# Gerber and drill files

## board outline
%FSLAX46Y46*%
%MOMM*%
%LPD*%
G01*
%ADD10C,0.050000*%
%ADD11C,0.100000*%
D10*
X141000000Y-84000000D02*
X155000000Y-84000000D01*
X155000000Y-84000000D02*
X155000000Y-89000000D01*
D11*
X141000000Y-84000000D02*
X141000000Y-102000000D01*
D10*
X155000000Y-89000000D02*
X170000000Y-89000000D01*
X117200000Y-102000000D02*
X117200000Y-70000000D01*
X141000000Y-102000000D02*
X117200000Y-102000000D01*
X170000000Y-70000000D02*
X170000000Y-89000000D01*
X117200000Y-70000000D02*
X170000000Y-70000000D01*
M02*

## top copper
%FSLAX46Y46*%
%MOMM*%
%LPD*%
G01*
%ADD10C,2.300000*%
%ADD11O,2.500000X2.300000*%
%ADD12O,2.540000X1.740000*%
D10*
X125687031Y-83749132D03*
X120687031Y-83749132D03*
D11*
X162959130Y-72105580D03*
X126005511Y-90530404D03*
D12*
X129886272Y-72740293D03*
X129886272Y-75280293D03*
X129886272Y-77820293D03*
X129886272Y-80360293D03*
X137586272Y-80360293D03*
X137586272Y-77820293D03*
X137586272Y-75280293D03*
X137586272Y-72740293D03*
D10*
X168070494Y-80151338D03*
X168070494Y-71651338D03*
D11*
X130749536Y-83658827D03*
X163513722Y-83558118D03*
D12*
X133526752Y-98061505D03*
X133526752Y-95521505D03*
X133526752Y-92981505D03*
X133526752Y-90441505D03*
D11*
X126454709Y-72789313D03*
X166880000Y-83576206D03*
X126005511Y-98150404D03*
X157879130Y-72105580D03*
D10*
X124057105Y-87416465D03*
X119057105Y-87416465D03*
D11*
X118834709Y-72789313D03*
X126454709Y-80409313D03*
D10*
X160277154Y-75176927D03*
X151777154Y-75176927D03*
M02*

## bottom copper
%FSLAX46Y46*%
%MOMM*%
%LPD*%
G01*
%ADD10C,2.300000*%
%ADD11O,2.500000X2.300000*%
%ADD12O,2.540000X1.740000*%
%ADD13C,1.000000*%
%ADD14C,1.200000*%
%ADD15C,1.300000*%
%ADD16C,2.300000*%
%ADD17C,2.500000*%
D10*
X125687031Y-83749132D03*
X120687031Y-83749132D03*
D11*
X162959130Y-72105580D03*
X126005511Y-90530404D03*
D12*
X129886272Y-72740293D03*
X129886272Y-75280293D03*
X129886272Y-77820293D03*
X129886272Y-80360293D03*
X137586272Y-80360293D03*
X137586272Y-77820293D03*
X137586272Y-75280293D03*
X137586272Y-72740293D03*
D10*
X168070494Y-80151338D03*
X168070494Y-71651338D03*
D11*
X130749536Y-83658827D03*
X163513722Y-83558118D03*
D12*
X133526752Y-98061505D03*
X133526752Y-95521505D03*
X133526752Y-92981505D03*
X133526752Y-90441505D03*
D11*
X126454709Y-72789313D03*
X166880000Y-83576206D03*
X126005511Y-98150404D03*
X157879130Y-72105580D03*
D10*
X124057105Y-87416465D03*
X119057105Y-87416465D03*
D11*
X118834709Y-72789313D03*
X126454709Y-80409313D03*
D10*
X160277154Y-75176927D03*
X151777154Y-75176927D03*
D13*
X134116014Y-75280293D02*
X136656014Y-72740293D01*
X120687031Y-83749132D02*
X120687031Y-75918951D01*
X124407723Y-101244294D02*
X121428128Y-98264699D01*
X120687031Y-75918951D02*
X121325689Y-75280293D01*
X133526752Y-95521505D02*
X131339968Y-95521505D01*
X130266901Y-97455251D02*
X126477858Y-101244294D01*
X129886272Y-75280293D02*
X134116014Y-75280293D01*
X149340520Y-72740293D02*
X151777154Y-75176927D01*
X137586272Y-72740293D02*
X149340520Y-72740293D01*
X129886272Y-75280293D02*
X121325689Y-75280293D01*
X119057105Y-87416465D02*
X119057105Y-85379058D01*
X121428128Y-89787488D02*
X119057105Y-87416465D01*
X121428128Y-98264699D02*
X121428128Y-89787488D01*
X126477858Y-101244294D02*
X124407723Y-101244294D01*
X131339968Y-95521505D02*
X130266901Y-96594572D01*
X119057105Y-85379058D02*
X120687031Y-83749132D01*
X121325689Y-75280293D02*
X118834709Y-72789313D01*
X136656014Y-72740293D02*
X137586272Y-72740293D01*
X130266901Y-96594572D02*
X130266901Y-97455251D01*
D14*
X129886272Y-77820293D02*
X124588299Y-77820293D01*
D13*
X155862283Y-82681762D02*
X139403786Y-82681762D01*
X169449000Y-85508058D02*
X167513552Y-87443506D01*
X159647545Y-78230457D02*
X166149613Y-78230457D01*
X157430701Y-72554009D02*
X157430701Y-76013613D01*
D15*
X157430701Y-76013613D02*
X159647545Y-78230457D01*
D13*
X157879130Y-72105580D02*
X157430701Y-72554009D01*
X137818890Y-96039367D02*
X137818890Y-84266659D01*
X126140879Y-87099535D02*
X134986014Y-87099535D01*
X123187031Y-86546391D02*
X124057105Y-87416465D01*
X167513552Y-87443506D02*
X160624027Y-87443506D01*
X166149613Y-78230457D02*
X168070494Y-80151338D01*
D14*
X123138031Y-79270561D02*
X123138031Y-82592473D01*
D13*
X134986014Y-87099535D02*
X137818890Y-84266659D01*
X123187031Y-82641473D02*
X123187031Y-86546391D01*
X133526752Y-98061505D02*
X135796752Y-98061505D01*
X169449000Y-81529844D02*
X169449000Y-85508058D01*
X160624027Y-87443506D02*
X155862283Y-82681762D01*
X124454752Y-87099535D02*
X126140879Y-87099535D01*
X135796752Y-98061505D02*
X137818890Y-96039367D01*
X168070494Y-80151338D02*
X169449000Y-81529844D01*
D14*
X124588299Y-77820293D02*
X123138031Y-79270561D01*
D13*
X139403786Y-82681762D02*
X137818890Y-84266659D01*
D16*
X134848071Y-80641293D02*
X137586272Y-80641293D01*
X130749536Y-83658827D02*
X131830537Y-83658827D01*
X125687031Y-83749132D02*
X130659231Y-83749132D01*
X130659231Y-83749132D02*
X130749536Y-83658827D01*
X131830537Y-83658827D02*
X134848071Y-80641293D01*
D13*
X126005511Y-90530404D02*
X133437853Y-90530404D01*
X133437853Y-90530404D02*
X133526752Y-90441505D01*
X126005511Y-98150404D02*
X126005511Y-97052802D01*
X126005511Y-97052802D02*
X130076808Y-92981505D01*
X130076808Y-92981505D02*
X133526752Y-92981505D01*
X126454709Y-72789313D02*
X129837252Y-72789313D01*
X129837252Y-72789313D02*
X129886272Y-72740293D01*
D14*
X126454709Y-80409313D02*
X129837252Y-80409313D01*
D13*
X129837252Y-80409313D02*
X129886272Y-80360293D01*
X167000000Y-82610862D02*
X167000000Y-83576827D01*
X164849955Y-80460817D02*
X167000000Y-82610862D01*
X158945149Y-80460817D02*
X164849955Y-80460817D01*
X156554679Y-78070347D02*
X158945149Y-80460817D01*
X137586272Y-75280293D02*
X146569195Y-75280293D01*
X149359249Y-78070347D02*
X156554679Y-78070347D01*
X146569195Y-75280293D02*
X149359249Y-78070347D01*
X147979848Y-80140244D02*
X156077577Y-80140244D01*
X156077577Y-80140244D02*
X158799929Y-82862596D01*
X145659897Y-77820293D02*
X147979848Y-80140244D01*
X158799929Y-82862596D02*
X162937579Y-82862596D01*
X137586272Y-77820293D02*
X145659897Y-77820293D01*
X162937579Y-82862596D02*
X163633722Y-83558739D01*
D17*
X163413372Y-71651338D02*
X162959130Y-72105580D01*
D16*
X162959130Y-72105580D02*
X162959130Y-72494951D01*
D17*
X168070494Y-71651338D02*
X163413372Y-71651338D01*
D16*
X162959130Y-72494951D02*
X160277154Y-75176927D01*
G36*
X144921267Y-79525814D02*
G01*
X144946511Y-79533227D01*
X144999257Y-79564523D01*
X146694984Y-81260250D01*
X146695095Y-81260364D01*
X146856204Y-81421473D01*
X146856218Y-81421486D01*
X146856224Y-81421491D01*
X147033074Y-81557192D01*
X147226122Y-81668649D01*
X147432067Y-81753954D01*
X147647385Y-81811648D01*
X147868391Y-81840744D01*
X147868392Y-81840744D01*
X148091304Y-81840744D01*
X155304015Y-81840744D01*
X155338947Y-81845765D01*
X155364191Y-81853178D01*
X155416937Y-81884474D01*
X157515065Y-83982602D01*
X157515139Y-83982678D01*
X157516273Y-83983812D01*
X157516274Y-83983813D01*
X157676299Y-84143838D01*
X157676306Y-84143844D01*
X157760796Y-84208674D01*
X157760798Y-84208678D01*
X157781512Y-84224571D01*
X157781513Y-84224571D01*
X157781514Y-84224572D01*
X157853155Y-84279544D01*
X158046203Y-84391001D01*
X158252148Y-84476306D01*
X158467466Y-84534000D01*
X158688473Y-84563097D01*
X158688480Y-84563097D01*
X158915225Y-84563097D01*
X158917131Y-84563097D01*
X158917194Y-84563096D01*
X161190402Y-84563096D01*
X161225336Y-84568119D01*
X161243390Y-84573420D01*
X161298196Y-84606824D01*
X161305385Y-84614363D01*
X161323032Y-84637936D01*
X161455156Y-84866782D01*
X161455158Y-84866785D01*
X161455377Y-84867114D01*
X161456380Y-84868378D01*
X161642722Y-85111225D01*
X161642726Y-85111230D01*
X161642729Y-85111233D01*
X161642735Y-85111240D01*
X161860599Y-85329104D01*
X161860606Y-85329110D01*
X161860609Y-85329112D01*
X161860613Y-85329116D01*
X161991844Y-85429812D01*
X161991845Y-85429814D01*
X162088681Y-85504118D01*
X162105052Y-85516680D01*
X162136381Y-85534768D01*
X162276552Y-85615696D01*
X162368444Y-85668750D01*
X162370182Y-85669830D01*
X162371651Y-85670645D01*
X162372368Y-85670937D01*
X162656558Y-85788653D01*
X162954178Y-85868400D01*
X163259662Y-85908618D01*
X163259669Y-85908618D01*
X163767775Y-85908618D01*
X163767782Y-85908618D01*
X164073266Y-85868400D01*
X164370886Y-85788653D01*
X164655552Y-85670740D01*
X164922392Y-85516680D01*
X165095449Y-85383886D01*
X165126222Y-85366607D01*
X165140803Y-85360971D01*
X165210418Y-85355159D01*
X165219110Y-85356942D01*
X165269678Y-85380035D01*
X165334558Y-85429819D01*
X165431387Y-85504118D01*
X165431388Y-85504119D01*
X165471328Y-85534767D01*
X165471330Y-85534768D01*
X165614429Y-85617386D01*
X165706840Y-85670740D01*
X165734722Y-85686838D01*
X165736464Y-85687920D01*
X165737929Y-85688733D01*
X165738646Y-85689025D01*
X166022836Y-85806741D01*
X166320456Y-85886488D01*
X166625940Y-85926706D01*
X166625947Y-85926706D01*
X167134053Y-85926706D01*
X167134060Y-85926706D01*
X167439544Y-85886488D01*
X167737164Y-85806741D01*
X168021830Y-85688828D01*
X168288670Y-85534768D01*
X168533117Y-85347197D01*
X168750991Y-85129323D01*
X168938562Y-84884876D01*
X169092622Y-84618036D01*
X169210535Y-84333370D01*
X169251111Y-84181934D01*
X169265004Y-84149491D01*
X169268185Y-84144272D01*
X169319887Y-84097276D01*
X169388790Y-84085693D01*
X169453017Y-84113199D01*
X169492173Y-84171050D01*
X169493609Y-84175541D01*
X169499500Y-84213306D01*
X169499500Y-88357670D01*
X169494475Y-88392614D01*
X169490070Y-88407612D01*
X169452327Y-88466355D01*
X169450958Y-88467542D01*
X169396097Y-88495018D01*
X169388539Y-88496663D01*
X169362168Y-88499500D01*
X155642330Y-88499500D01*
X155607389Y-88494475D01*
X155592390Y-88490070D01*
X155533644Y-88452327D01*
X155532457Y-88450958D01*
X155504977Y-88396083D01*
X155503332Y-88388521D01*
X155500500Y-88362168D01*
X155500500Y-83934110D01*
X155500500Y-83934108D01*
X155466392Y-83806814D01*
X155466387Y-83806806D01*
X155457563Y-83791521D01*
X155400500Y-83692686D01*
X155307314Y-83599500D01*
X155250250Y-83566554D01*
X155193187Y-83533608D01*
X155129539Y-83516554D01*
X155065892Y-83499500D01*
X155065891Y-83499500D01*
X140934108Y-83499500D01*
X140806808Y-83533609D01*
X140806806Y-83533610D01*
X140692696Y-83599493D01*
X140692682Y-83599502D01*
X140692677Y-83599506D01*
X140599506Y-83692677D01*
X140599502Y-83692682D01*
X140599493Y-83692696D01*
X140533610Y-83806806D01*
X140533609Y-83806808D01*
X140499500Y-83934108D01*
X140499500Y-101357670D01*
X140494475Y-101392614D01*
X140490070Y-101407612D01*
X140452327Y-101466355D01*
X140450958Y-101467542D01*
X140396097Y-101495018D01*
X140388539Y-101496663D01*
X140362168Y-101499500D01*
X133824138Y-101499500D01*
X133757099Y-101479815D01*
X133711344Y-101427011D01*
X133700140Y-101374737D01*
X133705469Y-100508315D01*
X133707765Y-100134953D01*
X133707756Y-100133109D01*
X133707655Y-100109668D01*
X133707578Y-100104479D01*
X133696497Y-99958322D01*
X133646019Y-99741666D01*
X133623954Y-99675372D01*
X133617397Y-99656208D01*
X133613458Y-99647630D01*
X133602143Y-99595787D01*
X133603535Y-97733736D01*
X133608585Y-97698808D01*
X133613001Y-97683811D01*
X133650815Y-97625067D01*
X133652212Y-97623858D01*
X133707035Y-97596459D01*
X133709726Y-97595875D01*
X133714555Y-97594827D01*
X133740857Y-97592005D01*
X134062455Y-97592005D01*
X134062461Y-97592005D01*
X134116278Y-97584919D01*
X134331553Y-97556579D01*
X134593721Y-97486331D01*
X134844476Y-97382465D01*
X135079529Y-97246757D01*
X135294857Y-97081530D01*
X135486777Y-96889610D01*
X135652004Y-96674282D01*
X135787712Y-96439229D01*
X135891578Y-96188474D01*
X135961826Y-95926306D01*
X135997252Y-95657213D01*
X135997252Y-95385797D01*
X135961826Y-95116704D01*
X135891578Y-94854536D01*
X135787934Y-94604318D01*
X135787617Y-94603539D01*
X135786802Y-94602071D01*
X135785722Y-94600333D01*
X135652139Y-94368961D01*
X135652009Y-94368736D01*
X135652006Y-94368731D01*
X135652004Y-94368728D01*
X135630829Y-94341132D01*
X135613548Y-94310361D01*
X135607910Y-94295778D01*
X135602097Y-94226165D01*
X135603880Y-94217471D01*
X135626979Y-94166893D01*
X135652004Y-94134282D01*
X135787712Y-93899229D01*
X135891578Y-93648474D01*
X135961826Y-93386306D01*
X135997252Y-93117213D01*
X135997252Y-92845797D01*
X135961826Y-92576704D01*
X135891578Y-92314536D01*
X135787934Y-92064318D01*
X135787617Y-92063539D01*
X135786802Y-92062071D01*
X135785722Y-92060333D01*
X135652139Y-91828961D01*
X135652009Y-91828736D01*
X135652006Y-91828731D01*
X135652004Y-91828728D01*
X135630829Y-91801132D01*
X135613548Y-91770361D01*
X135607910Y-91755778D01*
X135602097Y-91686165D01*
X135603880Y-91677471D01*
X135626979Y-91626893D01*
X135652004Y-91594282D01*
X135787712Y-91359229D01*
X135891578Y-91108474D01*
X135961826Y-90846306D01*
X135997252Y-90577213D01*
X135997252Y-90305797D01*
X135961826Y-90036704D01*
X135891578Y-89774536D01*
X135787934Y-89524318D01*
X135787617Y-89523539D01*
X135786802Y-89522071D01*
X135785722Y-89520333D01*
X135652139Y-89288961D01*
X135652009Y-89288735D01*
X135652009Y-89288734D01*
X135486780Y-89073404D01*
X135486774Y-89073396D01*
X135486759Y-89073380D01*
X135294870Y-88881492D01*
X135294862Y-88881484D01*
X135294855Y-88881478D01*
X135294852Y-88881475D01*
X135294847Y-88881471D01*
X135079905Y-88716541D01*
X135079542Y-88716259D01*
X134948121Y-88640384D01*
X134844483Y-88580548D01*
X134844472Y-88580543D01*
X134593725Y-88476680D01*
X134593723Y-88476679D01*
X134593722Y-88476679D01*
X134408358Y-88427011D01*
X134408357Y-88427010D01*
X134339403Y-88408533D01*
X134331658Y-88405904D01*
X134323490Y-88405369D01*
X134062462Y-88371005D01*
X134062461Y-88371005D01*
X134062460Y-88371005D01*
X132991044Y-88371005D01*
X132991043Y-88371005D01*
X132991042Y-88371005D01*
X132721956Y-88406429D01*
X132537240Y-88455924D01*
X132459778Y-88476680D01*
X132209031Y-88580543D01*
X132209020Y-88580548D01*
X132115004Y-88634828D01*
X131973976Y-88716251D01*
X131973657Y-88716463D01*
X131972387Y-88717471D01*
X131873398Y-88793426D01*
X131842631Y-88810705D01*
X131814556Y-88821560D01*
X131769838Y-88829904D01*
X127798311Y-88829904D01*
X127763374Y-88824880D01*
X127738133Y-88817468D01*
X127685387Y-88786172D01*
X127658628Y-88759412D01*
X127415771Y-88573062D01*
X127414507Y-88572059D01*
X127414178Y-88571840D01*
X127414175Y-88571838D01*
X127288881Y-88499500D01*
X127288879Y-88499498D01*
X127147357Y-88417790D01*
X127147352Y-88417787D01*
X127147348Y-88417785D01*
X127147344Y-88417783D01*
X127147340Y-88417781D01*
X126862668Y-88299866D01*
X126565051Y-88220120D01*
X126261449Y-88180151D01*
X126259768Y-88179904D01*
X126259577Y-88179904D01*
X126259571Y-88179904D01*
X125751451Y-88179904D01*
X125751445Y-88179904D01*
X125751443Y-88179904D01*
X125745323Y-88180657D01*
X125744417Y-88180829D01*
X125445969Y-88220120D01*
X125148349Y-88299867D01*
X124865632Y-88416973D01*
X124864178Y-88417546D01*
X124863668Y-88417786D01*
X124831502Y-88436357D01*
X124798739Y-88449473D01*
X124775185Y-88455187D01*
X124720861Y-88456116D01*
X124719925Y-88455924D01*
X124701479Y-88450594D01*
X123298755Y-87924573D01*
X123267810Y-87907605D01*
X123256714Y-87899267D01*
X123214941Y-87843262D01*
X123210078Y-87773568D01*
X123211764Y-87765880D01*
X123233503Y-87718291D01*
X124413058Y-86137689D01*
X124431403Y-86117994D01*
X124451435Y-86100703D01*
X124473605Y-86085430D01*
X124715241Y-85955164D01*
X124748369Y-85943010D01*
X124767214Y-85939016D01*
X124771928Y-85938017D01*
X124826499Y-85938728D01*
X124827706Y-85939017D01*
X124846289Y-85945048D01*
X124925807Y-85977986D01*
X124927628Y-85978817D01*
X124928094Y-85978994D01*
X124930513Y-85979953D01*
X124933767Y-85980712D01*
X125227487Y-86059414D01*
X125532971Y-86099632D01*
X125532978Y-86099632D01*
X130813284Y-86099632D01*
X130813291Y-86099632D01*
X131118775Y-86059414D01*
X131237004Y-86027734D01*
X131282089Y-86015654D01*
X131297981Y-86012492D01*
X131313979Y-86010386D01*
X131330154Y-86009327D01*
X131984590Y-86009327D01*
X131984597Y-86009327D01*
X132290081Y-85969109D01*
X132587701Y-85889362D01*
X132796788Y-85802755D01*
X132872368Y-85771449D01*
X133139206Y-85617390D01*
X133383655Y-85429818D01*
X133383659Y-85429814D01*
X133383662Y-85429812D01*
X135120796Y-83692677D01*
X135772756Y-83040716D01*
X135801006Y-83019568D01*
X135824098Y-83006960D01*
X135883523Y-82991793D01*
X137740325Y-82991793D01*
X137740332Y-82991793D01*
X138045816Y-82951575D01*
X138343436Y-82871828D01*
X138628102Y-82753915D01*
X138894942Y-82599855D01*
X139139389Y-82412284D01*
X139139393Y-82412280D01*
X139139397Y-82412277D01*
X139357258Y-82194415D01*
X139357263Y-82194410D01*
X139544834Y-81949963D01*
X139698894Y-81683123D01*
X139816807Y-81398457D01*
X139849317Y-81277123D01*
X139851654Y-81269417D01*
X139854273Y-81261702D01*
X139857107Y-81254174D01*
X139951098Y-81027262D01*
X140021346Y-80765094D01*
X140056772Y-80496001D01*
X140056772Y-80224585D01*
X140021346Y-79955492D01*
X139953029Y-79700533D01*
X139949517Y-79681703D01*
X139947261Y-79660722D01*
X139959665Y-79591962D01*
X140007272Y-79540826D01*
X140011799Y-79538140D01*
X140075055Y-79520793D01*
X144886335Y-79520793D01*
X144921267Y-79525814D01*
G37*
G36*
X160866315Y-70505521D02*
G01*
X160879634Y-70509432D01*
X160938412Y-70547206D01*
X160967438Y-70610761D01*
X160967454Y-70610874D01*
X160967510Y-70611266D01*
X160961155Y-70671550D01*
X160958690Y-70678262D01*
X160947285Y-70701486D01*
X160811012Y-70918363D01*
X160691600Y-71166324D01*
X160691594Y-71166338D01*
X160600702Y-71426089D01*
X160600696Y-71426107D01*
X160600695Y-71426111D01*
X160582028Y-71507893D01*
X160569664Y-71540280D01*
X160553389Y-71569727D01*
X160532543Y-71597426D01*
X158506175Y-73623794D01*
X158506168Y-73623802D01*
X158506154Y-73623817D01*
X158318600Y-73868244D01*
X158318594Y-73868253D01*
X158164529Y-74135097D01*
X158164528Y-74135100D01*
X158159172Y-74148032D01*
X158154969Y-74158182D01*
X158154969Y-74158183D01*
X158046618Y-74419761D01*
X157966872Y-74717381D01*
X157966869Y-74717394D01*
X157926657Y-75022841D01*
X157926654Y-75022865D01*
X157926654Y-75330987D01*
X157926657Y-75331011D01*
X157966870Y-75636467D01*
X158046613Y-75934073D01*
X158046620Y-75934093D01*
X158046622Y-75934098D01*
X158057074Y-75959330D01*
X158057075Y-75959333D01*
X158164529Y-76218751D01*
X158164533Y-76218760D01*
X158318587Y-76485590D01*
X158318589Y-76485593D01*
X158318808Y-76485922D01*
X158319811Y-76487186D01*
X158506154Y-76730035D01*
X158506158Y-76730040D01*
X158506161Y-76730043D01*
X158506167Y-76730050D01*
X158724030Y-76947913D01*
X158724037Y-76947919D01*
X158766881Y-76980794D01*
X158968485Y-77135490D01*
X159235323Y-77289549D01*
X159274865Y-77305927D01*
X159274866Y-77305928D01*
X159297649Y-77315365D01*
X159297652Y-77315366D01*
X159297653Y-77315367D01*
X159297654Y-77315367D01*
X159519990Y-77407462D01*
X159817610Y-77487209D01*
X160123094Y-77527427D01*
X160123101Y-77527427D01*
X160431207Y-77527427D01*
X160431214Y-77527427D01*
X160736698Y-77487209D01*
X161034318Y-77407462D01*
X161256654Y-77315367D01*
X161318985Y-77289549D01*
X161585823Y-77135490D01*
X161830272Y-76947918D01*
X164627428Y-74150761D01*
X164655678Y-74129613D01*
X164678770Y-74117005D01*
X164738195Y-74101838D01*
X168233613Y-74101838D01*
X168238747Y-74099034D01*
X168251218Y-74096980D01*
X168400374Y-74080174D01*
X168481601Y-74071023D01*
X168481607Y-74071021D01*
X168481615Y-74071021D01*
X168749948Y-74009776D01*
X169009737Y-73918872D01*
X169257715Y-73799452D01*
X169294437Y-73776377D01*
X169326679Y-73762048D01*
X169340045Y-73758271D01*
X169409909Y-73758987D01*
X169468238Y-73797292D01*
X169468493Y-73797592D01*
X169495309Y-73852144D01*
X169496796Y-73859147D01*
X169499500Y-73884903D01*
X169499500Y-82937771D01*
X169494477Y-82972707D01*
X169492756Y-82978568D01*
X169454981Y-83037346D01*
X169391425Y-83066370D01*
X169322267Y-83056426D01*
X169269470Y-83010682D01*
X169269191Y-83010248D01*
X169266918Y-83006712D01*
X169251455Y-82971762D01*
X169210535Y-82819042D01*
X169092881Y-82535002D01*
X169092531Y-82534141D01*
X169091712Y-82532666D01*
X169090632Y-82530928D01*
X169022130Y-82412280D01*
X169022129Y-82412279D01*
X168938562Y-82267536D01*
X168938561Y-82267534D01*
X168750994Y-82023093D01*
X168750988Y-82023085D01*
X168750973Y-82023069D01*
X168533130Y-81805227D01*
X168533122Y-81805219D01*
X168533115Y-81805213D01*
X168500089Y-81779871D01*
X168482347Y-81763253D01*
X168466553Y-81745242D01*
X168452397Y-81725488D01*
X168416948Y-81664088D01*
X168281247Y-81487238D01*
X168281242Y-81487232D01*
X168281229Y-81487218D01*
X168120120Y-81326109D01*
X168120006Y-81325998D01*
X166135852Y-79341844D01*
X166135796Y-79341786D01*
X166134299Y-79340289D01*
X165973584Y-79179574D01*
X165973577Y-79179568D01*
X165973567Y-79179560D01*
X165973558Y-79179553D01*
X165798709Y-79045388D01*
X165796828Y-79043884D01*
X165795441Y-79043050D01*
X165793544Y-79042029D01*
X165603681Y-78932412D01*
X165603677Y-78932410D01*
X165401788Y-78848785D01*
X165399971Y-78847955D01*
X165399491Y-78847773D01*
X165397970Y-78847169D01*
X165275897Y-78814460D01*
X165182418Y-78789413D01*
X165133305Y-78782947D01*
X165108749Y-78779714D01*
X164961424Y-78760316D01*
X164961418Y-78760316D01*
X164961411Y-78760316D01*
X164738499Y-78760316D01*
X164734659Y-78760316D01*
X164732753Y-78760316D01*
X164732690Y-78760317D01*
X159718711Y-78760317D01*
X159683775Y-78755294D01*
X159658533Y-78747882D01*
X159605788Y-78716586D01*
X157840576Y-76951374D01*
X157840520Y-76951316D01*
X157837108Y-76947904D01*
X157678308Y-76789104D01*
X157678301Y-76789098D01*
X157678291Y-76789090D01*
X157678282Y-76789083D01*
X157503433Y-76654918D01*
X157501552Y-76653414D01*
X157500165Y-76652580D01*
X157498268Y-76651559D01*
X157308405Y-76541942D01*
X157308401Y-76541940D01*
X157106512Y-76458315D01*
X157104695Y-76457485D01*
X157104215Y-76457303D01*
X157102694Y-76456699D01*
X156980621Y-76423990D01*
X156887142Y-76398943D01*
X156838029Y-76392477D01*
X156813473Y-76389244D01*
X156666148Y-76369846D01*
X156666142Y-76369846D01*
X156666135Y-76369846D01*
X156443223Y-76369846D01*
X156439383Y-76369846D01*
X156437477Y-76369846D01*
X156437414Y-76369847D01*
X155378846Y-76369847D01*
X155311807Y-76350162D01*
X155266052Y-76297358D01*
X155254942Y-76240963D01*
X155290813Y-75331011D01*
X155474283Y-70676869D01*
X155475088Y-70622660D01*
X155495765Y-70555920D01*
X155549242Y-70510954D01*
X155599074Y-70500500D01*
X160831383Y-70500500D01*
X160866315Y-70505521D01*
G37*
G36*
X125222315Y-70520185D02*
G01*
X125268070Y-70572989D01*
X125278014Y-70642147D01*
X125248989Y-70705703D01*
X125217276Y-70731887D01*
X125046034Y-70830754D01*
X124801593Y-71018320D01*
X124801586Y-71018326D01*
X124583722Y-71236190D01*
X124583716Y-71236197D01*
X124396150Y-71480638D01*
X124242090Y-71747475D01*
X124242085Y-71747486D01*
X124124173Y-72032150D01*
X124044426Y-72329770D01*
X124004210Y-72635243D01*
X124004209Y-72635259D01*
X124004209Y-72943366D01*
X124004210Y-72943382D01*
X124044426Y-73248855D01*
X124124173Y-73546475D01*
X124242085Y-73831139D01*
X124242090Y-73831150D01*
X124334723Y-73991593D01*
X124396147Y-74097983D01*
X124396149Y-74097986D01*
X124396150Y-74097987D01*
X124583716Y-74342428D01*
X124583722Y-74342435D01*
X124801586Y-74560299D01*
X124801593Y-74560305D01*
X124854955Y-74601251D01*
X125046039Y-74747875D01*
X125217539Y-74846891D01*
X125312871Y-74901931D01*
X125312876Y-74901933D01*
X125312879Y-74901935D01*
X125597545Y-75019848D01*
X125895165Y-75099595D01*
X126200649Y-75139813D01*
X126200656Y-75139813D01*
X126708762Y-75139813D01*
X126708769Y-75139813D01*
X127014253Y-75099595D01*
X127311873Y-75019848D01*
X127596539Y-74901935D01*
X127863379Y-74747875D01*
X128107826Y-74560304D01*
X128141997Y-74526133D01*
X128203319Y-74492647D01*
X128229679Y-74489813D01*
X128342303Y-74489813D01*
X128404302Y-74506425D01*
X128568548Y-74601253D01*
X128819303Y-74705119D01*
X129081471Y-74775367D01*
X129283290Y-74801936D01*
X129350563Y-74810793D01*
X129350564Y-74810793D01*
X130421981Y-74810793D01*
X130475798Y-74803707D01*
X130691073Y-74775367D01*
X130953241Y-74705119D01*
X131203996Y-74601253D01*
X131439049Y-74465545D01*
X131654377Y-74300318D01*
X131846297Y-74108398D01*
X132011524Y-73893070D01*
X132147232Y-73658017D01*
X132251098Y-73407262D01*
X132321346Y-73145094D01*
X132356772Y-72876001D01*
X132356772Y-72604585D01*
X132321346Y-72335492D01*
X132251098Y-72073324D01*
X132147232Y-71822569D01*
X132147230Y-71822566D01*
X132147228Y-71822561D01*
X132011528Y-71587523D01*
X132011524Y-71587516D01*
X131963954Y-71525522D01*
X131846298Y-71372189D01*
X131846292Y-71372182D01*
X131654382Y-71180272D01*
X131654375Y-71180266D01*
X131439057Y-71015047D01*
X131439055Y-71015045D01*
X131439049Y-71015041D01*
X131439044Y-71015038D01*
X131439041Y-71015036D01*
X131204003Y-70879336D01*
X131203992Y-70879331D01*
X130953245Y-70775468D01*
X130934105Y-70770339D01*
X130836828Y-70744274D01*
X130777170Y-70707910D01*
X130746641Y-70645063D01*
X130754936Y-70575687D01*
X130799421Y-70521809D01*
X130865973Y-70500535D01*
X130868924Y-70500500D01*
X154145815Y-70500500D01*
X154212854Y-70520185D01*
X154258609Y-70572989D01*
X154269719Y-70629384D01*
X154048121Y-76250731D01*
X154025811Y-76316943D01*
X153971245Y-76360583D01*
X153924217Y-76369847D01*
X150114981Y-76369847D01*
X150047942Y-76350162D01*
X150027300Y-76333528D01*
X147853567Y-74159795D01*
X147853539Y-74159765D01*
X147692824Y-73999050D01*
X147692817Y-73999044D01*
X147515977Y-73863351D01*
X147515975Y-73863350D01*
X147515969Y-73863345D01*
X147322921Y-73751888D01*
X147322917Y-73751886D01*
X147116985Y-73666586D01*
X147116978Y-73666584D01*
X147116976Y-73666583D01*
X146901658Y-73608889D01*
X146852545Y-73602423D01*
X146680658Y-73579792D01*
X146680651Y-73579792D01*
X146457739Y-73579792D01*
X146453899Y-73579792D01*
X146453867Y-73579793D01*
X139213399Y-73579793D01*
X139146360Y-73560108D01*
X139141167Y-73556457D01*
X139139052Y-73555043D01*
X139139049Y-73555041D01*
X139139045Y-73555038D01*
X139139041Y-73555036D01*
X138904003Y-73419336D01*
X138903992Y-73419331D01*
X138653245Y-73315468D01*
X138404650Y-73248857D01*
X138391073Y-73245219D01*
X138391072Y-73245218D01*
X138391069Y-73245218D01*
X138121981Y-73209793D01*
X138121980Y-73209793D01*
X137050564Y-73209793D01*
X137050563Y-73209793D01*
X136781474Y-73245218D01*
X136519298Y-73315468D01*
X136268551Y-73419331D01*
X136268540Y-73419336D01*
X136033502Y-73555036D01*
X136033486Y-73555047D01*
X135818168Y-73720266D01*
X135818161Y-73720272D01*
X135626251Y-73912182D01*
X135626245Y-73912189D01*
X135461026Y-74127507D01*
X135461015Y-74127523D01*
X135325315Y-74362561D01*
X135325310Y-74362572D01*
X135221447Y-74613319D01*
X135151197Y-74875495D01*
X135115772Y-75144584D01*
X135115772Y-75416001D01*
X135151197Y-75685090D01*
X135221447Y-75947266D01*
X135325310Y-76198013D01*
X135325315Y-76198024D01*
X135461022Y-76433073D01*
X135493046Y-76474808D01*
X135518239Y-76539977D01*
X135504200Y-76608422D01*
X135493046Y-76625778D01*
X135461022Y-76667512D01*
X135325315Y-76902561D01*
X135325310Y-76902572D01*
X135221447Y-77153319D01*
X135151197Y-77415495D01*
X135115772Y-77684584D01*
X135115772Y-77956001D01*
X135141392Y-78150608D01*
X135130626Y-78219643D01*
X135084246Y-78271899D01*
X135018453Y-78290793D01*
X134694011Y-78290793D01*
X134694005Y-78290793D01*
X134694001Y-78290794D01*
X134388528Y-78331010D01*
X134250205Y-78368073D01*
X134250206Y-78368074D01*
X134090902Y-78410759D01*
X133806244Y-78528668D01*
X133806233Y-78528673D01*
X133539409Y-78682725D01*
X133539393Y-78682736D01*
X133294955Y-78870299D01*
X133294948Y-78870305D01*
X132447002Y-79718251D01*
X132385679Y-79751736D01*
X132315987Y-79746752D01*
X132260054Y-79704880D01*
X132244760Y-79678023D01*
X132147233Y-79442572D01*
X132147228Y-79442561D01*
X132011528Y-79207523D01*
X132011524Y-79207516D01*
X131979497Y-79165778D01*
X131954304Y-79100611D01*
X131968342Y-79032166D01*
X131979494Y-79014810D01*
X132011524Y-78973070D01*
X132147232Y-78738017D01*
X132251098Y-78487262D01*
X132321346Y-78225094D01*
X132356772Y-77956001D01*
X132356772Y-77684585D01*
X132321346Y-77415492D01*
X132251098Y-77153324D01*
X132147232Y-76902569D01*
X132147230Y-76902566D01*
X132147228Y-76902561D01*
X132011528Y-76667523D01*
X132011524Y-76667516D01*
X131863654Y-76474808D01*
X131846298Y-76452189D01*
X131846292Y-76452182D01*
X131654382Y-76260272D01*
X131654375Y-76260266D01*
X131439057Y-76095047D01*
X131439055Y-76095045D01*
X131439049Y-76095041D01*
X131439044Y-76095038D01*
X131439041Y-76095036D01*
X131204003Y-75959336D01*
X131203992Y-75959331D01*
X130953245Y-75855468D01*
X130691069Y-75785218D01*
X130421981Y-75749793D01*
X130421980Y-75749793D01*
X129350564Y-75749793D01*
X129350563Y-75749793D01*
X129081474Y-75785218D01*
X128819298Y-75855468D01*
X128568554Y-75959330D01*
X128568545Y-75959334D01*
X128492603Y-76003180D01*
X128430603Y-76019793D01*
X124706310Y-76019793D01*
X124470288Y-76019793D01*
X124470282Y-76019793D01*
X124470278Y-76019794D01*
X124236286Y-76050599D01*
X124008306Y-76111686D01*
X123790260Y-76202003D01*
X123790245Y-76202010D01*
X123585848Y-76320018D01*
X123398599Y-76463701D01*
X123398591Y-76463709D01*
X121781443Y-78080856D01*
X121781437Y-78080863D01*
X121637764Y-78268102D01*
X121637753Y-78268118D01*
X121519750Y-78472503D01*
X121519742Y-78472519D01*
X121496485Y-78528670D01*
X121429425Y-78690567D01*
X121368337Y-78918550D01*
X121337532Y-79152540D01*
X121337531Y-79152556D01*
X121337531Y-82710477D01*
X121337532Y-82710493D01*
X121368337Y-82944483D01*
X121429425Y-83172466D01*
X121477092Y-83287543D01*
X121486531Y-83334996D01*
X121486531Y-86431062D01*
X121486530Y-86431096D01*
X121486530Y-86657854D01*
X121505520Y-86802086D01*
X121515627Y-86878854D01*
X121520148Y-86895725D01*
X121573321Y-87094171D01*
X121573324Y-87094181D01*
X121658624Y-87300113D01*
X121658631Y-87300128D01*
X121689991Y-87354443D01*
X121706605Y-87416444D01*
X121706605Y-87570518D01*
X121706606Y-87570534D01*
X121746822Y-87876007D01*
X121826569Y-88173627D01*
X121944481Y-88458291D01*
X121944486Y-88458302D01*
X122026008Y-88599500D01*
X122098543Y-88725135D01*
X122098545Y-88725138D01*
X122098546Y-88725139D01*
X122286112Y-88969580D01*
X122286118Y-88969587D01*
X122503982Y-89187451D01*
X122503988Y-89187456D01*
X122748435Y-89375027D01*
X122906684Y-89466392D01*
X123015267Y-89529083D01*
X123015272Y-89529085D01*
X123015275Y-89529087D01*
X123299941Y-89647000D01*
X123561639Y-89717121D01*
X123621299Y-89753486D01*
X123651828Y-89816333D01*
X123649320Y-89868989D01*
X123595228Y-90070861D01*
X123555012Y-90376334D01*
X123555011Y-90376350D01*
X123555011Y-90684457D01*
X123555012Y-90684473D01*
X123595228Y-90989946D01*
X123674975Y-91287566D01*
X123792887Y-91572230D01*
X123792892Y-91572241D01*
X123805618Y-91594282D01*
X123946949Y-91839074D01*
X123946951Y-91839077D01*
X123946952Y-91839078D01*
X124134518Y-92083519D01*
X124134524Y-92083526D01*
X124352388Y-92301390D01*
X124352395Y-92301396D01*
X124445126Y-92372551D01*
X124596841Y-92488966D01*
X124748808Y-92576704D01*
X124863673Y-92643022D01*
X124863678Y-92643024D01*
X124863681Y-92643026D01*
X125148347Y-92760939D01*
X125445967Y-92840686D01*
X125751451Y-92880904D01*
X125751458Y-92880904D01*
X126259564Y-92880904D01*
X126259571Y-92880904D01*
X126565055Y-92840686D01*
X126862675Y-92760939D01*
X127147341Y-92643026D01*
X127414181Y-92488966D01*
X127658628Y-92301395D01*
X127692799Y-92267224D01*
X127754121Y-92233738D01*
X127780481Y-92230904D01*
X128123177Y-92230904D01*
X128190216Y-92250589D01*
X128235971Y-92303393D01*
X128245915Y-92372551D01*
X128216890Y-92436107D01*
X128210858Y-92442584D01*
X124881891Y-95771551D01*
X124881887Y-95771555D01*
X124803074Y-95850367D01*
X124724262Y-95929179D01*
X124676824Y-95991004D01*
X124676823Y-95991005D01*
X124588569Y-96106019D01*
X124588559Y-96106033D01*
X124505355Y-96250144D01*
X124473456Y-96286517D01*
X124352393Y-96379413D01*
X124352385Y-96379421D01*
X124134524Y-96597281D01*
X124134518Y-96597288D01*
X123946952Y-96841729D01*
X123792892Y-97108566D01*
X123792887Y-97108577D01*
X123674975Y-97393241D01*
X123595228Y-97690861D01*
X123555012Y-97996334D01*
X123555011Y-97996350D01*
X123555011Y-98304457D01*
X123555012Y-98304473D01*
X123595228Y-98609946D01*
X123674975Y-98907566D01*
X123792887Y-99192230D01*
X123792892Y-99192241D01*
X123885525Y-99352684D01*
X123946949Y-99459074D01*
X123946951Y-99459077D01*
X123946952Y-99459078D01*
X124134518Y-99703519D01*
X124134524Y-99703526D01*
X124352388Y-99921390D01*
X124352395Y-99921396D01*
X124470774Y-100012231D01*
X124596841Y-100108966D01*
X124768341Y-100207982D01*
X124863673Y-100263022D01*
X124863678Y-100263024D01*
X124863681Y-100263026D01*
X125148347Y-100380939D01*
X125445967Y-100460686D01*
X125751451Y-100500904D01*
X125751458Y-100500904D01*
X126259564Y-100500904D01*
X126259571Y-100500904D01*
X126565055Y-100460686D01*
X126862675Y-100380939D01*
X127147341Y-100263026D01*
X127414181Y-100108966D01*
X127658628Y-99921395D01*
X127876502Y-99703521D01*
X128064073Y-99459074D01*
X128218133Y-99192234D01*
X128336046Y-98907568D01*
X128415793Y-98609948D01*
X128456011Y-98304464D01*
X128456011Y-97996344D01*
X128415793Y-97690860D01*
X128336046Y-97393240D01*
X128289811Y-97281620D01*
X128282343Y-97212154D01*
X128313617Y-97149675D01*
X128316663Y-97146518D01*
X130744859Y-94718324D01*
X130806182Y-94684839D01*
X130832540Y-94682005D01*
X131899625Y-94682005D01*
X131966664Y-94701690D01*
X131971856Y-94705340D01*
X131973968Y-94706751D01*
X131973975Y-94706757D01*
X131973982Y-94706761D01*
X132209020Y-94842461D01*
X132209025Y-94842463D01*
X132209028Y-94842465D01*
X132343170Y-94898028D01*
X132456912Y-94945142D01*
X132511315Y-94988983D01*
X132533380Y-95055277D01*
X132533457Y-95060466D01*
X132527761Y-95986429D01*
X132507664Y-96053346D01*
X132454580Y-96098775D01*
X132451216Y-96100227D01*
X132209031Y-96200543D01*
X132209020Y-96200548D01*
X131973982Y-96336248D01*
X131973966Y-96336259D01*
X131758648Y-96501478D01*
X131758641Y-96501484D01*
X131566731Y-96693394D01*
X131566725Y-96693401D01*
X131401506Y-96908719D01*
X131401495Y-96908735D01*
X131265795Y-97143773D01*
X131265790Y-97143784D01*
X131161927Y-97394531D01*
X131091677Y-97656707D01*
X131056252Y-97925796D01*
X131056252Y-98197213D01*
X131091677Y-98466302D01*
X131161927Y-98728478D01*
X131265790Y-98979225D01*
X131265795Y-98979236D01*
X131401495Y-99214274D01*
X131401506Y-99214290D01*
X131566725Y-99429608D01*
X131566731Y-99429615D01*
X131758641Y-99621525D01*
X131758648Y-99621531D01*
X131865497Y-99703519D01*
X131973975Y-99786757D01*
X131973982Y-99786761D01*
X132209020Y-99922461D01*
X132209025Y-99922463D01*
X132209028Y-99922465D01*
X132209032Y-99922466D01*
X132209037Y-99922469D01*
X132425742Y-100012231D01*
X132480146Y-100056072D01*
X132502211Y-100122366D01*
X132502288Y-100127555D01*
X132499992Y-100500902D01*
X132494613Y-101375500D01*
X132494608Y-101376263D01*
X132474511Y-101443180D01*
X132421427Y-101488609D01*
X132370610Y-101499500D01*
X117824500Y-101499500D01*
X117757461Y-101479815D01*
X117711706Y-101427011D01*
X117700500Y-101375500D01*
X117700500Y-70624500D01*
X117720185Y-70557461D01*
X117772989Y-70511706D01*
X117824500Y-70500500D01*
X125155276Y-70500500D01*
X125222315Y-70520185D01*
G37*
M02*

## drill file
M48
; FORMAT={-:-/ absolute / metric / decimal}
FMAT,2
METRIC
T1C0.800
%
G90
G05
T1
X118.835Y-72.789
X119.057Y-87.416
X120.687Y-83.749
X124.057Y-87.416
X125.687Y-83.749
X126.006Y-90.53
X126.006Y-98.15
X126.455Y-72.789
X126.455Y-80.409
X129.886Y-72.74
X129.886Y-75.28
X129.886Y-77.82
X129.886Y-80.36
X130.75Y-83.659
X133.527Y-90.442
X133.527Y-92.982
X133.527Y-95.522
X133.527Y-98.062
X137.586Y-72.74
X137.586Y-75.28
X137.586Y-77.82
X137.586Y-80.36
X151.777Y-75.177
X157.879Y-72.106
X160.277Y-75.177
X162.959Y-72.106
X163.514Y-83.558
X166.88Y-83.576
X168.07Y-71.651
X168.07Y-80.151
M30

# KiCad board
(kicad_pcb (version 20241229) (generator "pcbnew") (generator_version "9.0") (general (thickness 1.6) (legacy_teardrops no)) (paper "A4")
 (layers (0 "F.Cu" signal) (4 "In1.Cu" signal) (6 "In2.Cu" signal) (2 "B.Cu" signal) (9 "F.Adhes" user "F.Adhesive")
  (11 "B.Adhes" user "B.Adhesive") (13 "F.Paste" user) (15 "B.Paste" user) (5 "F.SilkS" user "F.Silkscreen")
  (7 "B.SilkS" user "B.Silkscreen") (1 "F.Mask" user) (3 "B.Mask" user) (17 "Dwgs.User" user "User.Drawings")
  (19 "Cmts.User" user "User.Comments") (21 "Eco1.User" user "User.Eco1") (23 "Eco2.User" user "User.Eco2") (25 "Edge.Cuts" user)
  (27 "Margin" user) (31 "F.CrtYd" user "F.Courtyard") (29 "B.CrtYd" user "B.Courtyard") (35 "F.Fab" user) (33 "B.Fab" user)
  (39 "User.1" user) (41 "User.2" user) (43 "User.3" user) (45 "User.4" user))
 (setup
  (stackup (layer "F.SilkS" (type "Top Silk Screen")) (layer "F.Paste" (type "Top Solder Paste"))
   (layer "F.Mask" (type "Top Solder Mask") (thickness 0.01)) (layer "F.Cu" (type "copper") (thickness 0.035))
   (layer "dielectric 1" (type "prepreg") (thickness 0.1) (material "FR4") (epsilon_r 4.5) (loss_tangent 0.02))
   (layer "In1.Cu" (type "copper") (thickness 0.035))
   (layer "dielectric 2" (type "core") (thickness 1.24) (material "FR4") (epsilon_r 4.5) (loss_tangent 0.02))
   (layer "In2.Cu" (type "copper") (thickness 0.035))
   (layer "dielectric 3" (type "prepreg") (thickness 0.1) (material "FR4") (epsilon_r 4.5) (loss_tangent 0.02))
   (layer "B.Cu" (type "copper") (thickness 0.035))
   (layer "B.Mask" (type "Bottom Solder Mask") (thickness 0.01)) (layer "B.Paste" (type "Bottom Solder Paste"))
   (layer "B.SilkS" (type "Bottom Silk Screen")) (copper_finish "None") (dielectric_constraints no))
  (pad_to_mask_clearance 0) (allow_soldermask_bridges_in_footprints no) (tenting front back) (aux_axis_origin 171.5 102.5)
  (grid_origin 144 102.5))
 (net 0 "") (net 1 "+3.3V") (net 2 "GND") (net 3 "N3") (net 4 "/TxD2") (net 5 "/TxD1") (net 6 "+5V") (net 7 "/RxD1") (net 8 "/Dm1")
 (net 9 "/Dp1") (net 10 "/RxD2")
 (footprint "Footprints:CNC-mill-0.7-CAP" (layer "F.Cu") (at 123.187031 83.749132 90)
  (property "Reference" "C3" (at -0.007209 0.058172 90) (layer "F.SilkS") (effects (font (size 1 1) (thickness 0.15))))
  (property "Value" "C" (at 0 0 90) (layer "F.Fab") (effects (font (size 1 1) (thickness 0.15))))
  (pad "1" thru_hole circle (at 0 2.5 90) (size 2.3 2.3) (drill 0.8) (layers "*.Cu" "*.Mask") (remove_unused_layers no) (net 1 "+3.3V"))
  (pad "2" thru_hole circle (at 0 -2.5 90) (size 2.3 2.3) (drill 0.8) (layers "*.Cu" "*.Mask") (remove_unused_layers no) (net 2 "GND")))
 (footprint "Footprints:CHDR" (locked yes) (layer "F.Cu") (at 162.95913 72.10558)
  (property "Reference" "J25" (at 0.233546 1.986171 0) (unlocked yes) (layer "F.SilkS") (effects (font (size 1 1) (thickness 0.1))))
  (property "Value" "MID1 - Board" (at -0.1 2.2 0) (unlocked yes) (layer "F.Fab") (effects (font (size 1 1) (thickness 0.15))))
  (pad "1" thru_hole oval (at 0 0) (size 2.5 2.3) (drill 0.8) (layers "*.Cu" "*.Mask") (remove_unused_layers no) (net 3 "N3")))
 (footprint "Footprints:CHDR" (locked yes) (layer "F.Cu") (at 126.005511 90.530404)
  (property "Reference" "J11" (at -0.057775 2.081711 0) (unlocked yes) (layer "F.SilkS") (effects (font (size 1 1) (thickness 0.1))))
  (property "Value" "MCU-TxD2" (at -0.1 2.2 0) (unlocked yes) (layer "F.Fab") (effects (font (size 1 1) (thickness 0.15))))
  (pad "1" thru_hole oval (at 0 0) (size 2.5 2.3) (drill 0.8) (layers "*.Cu" "*.Mask") (remove_unused_layers no) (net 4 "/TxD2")))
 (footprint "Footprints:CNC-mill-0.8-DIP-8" (layer "F.Cu") (at 133.736272 76.550293 -90)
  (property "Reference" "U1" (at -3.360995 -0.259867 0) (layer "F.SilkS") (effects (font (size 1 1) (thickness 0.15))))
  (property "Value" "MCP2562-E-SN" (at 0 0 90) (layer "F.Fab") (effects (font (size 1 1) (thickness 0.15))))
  (pad "1" thru_hole oval (at -3.81 3.85 270) (size 1.74 2.54) (drill 0.8) (layers "*.Cu" "*.Mask") (remove_unused_layers no)
   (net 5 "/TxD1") (thermal_bridge_angle 45))
  (pad "2" thru_hole oval (at -1.27 3.85 270) (size 1.74 2.54) (drill 0.8) (layers "*.Cu" "*.Mask") (remove_unused_layers no) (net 2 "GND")
   (thermal_bridge_angle 45))
  (pad "3" thru_hole oval (at 1.27 3.85 270) (size 1.74 2.54) (drill 0.8) (layers "*.Cu" "*.Mask") (remove_unused_layers no) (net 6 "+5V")
   (thermal_bridge_angle 45))
  (pad "4" thru_hole oval (at 3.81 3.85 270) (size 1.74 2.54) (drill 0.8) (layers "*.Cu" "*.Mask") (remove_unused_layers no) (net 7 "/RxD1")
   (thermal_bridge_angle 45))
  (pad "5" thru_hole oval (at 3.81 -3.85 270) (size 1.74 2.54) (drill 0.8) (layers "*.Cu" "*.Mask") (remove_unused_layers no)
   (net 1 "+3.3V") (thermal_bridge_angle 45))
  (pad "6" thru_hole oval (at 1.27 -3.85 270) (size 1.74 2.54) (drill 0.8) (layers "*.Cu" "*.Mask") (remove_unused_layers no) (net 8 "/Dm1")
   (thermal_bridge_angle 45))
  (pad "7" thru_hole oval (at -1.27 -3.85 270) (size 1.74 2.54) (drill 0.8) (layers "*.Cu" "*.Mask") (remove_unused_layers no)
   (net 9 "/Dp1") (thermal_bridge_angle 45))
  (pad "8" thru_hole oval (at -3.81 -3.85 270) (size 1.74 2.54) (drill 0.8) (layers "*.Cu" "*.Mask") (remove_unused_layers no) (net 2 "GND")
   (thermal_bridge_angle 45)))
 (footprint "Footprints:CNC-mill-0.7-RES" (layer "F.Cu") (at 168.070494 75.901338)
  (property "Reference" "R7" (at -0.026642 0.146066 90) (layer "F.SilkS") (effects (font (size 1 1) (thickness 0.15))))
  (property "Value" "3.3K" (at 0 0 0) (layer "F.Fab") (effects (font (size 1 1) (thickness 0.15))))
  (pad "1" thru_hole circle (at 0 4.25) (size 2.3 2.3) (drill 0.8) (layers "*.Cu" "*.Mask") (remove_unused_layers no) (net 6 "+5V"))
  (pad "2" thru_hole circle (at 0 -4.25) (size 2.3 2.3) (drill 0.8) (layers "*.Cu" "*.Mask") (remove_unused_layers no) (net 3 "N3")))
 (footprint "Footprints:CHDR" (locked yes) (layer "F.Cu") (at 130.749536 83.658827)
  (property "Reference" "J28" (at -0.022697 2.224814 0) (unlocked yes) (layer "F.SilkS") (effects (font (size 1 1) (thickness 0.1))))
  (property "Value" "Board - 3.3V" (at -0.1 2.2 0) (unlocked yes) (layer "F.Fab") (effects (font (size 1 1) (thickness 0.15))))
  (pad "1" thru_hole oval (at 0 0) (size 2.5 2.3) (drill 0.8) (layers "*.Cu" "*.Mask") (remove_unused_layers no) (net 1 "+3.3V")))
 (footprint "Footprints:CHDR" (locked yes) (layer "F.Cu") (at 163.513722 83.558118)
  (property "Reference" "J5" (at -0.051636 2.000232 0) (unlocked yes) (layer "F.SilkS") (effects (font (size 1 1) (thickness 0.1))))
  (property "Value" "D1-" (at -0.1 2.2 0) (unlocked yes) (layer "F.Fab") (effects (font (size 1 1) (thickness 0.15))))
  (pad "1" thru_hole oval (at 0 0) (size 2.5 2.3) (drill 0.8) (layers "*.Cu" "*.Mask") (remove_unused_layers no) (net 8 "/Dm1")))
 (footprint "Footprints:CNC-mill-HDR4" (layer "F.Cu") (at 133.526752 98.061505 90)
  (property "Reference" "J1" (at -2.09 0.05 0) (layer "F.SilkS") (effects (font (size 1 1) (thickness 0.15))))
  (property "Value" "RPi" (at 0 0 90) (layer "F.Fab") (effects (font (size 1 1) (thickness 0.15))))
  (pad "1" thru_hole oval (at 0 0 90) (size 1.74 2.54) (drill 0.8) (layers "*.Cu" "*.Mask") (remove_unused_layers no) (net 6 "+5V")
   (thermal_bridge_angle 45))
  (pad "2" thru_hole oval (at 2.54 0 90) (size 1.74 2.54) (drill 0.8) (layers "*.Cu" "*.Mask") (remove_unused_layers no) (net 2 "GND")
   (thermal_bridge_angle 45))
  (pad "3" thru_hole oval (at 5.08 0 90) (size 1.74 2.54) (drill 0.8) (layers "*.Cu" "*.Mask") (remove_unused_layers no) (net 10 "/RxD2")
   (thermal_bridge_angle 45))
  (pad "4" thru_hole oval (at 7.62 0 90) (size 1.74 2.54) (drill 0.8) (layers "*.Cu" "*.Mask") (remove_unused_layers no) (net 4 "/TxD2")
   (thermal_bridge_angle 45)))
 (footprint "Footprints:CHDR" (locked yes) (layer "F.Cu") (at 126.454709 72.789313)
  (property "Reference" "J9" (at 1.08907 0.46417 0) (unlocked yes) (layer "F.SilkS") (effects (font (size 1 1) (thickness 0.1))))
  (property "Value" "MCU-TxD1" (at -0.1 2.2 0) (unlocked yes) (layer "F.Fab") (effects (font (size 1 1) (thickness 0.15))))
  (pad "1" thru_hole oval (at 0 0) (size 2.5 2.3) (drill 0.8) (layers "*.Cu" "*.Mask") (remove_unused_layers no) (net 5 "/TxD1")))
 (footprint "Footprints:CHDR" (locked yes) (layer "F.Cu") (at 166.88 83.576206)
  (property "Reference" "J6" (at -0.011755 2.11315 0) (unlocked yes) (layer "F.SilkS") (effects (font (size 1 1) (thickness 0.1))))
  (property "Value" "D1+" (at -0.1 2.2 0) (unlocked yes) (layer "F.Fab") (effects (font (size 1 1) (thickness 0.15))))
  (pad "1" thru_hole oval (at 0 0) (size 2.5 2.3) (drill 0.8) (layers "*.Cu" "*.Mask") (remove_unused_layers no) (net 9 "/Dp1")))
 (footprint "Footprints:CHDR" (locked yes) (layer "F.Cu") (at 126.005511 98.150404)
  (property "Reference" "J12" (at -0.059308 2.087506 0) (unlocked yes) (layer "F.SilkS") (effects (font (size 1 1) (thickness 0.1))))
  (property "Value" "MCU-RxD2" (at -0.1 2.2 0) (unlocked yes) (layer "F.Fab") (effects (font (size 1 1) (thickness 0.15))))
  (pad "1" thru_hole oval (at 0 0) (size 2.5 2.3) (drill 0.8) (layers "*.Cu" "*.Mask") (remove_unused_layers no) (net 10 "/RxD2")))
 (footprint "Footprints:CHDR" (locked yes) (layer "F.Cu") (at 157.87913 72.10558)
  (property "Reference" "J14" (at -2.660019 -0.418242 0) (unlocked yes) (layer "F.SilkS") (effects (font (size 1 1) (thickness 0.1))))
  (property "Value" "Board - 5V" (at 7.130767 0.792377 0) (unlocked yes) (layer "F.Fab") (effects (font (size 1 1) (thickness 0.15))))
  (pad "1" thru_hole oval (at 0 0) (size 2.5 2.3) (drill 0.8) (layers "*.Cu" "*.Mask") (remove_unused_layers no) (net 6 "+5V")))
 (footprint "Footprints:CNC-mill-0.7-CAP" (layer "F.Cu") (at 121.557105 87.416465 90)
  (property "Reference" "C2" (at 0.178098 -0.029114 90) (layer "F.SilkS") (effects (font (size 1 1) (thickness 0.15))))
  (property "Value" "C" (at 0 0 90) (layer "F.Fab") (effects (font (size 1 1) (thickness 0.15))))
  (pad "1" thru_hole circle (at 0 2.5 90) (size 2.3 2.3) (drill 0.8) (layers "*.Cu" "*.Mask") (remove_unused_layers no) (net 6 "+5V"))
  (pad "2" thru_hole circle (at 0 -2.5 90) (size 2.3 2.3) (drill 0.8) (layers "*.Cu" "*.Mask") (remove_unused_layers no) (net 2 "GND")))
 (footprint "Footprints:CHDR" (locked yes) (layer "F.Cu") (at 118.834709 72.789313)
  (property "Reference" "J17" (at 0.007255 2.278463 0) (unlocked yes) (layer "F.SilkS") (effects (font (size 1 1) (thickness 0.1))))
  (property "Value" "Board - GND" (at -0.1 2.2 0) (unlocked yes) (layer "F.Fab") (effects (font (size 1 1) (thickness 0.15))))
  (pad "1" thru_hole oval (at 0 0) (size 2.5 2.3) (drill 0.8) (layers "*.Cu" "*.Mask") (remove_unused_layers no) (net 2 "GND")))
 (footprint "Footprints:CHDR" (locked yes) (layer "F.Cu") (at 126.454709 80.409313)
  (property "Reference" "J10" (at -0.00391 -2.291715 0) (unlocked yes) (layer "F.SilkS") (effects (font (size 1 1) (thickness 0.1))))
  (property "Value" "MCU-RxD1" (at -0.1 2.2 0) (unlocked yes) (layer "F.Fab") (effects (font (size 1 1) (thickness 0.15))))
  (pad "1" thru_hole oval (at 0 0) (size 2.5 2.3) (drill 0.8) (layers "*.Cu" "*.Mask") (remove_unused_layers no) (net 7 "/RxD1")))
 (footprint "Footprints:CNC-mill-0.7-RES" (layer "F.Cu") (at 156.027154 75.176927 90)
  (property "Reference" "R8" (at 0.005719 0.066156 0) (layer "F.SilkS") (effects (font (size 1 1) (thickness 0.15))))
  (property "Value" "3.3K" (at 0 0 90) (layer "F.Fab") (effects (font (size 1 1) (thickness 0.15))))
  (pad "1" thru_hole circle (at 0 4.25 90) (size 2.3 2.3) (drill 0.8) (layers "*.Cu" "*.Mask") (remove_unused_layers no) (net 3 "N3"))
  (pad "2" thru_hole circle (at 0 -4.25 90) (size 2.3 2.3) (drill 0.8) (layers "*.Cu" "*.Mask") (remove_unused_layers no) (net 2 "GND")))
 (gr_line (start 141 84) (end 155 84) (stroke (width 0.05) (type default)) (locked yes) (layer "Edge.Cuts"))
 (gr_line (start 155 84) (end 155 89) (stroke (width 0.05) (type default)) (locked yes) (layer "Edge.Cuts"))
 (gr_line (start 141 84) (end 141 102) (stroke (width 0) (type default)) (locked yes) (layer "Edge.Cuts"))
 (gr_line (start 155 89) (end 170 89) (stroke (width 0.05) (type default)) (locked yes) (layer "Edge.Cuts"))
 (gr_line (start 117.2 102) (end 117.2 70) (stroke (width 0.05) (type default)) (locked yes) (layer "Edge.Cuts"))
 (gr_line (start 141 102) (end 117.2 102) (stroke (width 0.05) (type default)) (locked yes) (layer "Edge.Cuts"))
 (gr_line (start 170 70) (end 170 89) (stroke (width 0.05) (type default)) (locked yes) (layer "Edge.Cuts"))
 (gr_line (start 117.2 70) (end 170 70) (stroke (width 0.05) (type default)) (locked yes) (layer "Edge.Cuts"))
 (segment (start 134.116014 75.280293) (end 136.656014 72.740293) (width 1) (layer "B.Cu") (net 2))
 (segment (start 120.687031 83.749132) (end 120.687031 75.918951) (width 1) (layer "B.Cu") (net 2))
 (segment (start 124.407723 101.244294) (end 121.428128 98.264699) (width 1) (layer "B.Cu") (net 2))
 (segment (start 120.687031 75.918951) (end 121.325689 75.280293) (width 1) (layer "B.Cu") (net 2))
 (segment (start 133.526752 95.521505) (end 131.339968 95.521505) (width 1) (layer "B.Cu") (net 2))
 (segment (start 130.266901 97.455251) (end 126.477858 101.244294) (width 1) (layer "B.Cu") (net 2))
 (segment (start 129.886272 75.280293) (end 134.116014 75.280293) (width 1) (layer "B.Cu") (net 2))
 (segment (start 149.34052 72.740293) (end 151.777154 75.176927) (width 1) (layer "B.Cu") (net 2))
 (segment (start 137.586272 72.740293) (end 149.34052 72.740293) (width 1) (layer "B.Cu") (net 2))
 (segment (start 129.886272 75.280293) (end 121.325689 75.280293) (width 1) (layer "B.Cu") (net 2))
 (segment (start 119.057105 87.416465) (end 119.057105 85.379058) (width 1) (layer "B.Cu") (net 2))
 (segment (start 121.428128 89.787488) (end 119.057105 87.416465) (width 1) (layer "B.Cu") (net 2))
 (segment (start 121.428128 98.264699) (end 121.428128 89.787488) (width 1) (layer "B.Cu") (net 2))
 (segment (start 126.477858 101.244294) (end 124.407723 101.244294) (width 1) (layer "B.Cu") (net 2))
 (segment (start 131.339968 95.521505) (end 130.266901 96.594572) (width 1) (layer "B.Cu") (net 2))
 (segment (start 119.057105 85.379058) (end 120.687031 83.749132) (width 1) (layer "B.Cu") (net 2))
 (segment (start 121.325689 75.280293) (end 118.834709 72.789313) (width 1) (layer "B.Cu") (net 2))
 (segment (start 136.656014 72.740293) (end 137.586272 72.740293) (width 1) (layer "B.Cu") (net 2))
 (segment (start 130.266901 96.594572) (end 130.266901 97.455251) (width 1) (layer "B.Cu") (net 2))
 (segment (start 129.886272 77.820293) (end 124.588299 77.820293) (width 1.2) (layer "B.Cu") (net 6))
 (segment (start 155.862283 82.681762) (end 139.403786 82.681762) (width 1) (layer "B.Cu") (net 6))
 (segment (start 169.449 85.508058) (end 167.513552 87.443506) (width 1) (layer "B.Cu") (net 6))
 (segment (start 159.647545 78.230457) (end 166.149613 78.230457) (width 1) (layer "B.Cu") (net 6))
 (segment (start 157.430701 72.554009) (end 157.430701 76.013613) (width 1) (layer "B.Cu") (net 6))
 (segment (start 157.430701 76.013613) (end 159.647545 78.230457) (width 1.3) (layer "B.Cu") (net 6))
 (segment (start 157.87913 72.10558) (end 157.430701 72.554009) (width 1) (layer "B.Cu") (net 6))
 (segment (start 137.81889 96.039367) (end 137.81889 84.266659) (width 1) (layer "B.Cu") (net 6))
 (segment (start 126.140879 87.099535) (end 134.986014 87.099535) (width 1) (layer "B.Cu") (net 6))
 (segment (start 123.187031 86.546391) (end 124.057105 87.416465) (width 1) (layer "B.Cu") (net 6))
 (segment (start 167.513552 87.443506) (end 160.624027 87.443506) (width 1) (layer "B.Cu") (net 6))
 (segment (start 166.149613 78.230457) (end 168.070494 80.151338) (width 1) (layer "B.Cu") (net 6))
 (segment (start 123.138031 79.270561) (end 123.138031 82.592473) (width 1.2) (layer "B.Cu") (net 6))
 (segment (start 134.986014 87.099535) (end 137.81889 84.266659) (width 1) (layer "B.Cu") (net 6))
 (segment (start 123.187031 82.641473) (end 123.187031 86.546391) (width 1) (layer "B.Cu") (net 6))
 (segment (start 133.526752 98.061505) (end 135.796752 98.061505) (width 1) (layer "B.Cu") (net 6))
 (segment (start 169.449 81.529844) (end 169.449 85.508058) (width 1) (layer "B.Cu") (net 6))
 (segment (start 160.624027 87.443506) (end 155.862283 82.681762) (width 1) (layer "B.Cu") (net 6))
 (segment (start 124.454752 87.099535) (end 126.140879 87.099535) (width 1) (layer "B.Cu") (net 6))
 (segment (start 135.796752 98.061505) (end 137.81889 96.039367) (width 1) (layer "B.Cu") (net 6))
 (segment (start 168.070494 80.151338) (end 169.449 81.529844) (width 1) (layer "B.Cu") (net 6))
 (segment (start 124.588299 77.820293) (end 123.138031 79.270561) (width 1.2) (layer "B.Cu") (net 6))
 (segment (start 139.403786 82.681762) (end 137.81889 84.266659) (width 1) (layer "B.Cu") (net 6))
 (segment (start 134.848071 80.641293) (end 137.586272 80.641293) (width 2.3) (layer "B.Cu") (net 1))
 (segment (start 130.749536 83.658827) (end 131.830537 83.658827) (width 2.3) (layer "B.Cu") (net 1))
 (segment (start 125.687031 83.749132) (end 130.659231 83.749132) (width 2.3) (layer "B.Cu") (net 1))
 (segment (start 130.659231 83.749132) (end 130.749536 83.658827) (width 2.3) (layer "B.Cu") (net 1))
 (segment (start 131.830537 83.658827) (end 134.848071 80.641293) (width 2.3) (layer "B.Cu") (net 1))
 (segment (start 126.005511 90.530404) (end 133.437853 90.530404) (width 1) (layer "B.Cu") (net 4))
 (segment (start 133.437853 90.530404) (end 133.526752 90.441505) (width 1) (layer "B.Cu") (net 4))
 (segment (start 126.005511 98.150404) (end 126.005511 97.052802) (width 1) (layer "B.Cu") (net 10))
 (segment (start 126.005511 97.052802) (end 130.076808 92.981505) (width 1) (layer "B.Cu") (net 10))
 (segment (start 130.076808 92.981505) (end 133.526752 92.981505) (width 1) (layer "B.Cu") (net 10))
 (segment (start 126.454709 72.789313) (end 129.837252 72.789313) (width 1) (layer "B.Cu") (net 5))
 (segment (start 129.837252 72.789313) (end 129.886272 72.740293) (width 1) (layer "B.Cu") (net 5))
 (segment (start 126.454709 80.409313) (end 129.837252 80.409313) (width 1.2) (layer "B.Cu") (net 7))
 (segment (start 129.837252 80.409313) (end 129.886272 80.360293) (width 1) (layer "B.Cu") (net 7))
 (segment (start 167 82.610862) (end 167 83.576827) (width 1) (layer "B.Cu") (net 9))
 (segment (start 164.849955 80.460817) (end 167 82.610862) (width 1) (layer "B.Cu") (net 9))
 (segment (start 158.945149 80.460817) (end 164.849955 80.460817) (width 1) (layer "B.Cu") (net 9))
 (segment (start 156.554679 78.070347) (end 158.945149 80.460817) (width 1) (layer "B.Cu") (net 9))
 (segment (start 137.586272 75.280293) (end 146.569195 75.280293) (width 1) (layer "B.Cu") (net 9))
 (segment (start 149.359249 78.070347) (end 156.554679 78.070347) (width 1) (layer "B.Cu") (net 9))
 (segment (start 146.569195 75.280293) (end 149.359249 78.070347) (width 1) (layer "B.Cu") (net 9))
 (segment (start 147.979848 80.140244) (end 156.077577 80.140244) (width 1) (layer "B.Cu") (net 8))
 (segment (start 156.077577 80.140244) (end 158.799929 82.862596) (width 1) (layer "B.Cu") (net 8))
 (segment (start 145.659897 77.820293) (end 147.979848 80.140244) (width 1) (layer "B.Cu") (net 8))
 (segment (start 158.799929 82.862596) (end 162.937579 82.862596) (width 1) (layer "B.Cu") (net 8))
 (segment (start 137.586272 77.820293) (end 145.659897 77.820293) (width 1) (layer "B.Cu") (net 8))
 (segment (start 162.937579 82.862596) (end 163.633722 83.558739) (width 1) (layer "B.Cu") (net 8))
 (segment (start 163.413372 71.651338) (end 162.95913 72.10558) (width 2.5) (layer "B.Cu") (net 3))
 (segment (start 162.95913 72.10558) (end 162.95913 72.494951) (width 2.3) (layer "B.Cu") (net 3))
 (segment (start 168.070494 71.651338) (end 163.413372 71.651338) (width 2.5) (layer "B.Cu") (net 3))
 (segment (start 162.95913 72.494951) (end 160.277154 75.176927) (width 2.3) (layer "B.Cu") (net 3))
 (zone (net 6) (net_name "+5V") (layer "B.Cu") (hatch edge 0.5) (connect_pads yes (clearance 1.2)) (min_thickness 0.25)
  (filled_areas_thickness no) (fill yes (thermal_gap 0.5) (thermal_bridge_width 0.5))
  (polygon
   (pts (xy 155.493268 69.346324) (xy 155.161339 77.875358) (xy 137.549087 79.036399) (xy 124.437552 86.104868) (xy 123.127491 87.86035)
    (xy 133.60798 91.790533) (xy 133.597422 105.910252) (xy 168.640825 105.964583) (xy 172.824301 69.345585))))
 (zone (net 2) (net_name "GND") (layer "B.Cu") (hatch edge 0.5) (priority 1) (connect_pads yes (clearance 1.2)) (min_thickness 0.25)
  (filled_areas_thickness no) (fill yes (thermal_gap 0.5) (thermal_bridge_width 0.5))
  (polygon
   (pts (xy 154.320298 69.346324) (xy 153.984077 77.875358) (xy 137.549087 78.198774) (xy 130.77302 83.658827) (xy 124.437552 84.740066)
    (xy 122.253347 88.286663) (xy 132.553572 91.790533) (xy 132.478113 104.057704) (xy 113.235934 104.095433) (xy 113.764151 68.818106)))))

